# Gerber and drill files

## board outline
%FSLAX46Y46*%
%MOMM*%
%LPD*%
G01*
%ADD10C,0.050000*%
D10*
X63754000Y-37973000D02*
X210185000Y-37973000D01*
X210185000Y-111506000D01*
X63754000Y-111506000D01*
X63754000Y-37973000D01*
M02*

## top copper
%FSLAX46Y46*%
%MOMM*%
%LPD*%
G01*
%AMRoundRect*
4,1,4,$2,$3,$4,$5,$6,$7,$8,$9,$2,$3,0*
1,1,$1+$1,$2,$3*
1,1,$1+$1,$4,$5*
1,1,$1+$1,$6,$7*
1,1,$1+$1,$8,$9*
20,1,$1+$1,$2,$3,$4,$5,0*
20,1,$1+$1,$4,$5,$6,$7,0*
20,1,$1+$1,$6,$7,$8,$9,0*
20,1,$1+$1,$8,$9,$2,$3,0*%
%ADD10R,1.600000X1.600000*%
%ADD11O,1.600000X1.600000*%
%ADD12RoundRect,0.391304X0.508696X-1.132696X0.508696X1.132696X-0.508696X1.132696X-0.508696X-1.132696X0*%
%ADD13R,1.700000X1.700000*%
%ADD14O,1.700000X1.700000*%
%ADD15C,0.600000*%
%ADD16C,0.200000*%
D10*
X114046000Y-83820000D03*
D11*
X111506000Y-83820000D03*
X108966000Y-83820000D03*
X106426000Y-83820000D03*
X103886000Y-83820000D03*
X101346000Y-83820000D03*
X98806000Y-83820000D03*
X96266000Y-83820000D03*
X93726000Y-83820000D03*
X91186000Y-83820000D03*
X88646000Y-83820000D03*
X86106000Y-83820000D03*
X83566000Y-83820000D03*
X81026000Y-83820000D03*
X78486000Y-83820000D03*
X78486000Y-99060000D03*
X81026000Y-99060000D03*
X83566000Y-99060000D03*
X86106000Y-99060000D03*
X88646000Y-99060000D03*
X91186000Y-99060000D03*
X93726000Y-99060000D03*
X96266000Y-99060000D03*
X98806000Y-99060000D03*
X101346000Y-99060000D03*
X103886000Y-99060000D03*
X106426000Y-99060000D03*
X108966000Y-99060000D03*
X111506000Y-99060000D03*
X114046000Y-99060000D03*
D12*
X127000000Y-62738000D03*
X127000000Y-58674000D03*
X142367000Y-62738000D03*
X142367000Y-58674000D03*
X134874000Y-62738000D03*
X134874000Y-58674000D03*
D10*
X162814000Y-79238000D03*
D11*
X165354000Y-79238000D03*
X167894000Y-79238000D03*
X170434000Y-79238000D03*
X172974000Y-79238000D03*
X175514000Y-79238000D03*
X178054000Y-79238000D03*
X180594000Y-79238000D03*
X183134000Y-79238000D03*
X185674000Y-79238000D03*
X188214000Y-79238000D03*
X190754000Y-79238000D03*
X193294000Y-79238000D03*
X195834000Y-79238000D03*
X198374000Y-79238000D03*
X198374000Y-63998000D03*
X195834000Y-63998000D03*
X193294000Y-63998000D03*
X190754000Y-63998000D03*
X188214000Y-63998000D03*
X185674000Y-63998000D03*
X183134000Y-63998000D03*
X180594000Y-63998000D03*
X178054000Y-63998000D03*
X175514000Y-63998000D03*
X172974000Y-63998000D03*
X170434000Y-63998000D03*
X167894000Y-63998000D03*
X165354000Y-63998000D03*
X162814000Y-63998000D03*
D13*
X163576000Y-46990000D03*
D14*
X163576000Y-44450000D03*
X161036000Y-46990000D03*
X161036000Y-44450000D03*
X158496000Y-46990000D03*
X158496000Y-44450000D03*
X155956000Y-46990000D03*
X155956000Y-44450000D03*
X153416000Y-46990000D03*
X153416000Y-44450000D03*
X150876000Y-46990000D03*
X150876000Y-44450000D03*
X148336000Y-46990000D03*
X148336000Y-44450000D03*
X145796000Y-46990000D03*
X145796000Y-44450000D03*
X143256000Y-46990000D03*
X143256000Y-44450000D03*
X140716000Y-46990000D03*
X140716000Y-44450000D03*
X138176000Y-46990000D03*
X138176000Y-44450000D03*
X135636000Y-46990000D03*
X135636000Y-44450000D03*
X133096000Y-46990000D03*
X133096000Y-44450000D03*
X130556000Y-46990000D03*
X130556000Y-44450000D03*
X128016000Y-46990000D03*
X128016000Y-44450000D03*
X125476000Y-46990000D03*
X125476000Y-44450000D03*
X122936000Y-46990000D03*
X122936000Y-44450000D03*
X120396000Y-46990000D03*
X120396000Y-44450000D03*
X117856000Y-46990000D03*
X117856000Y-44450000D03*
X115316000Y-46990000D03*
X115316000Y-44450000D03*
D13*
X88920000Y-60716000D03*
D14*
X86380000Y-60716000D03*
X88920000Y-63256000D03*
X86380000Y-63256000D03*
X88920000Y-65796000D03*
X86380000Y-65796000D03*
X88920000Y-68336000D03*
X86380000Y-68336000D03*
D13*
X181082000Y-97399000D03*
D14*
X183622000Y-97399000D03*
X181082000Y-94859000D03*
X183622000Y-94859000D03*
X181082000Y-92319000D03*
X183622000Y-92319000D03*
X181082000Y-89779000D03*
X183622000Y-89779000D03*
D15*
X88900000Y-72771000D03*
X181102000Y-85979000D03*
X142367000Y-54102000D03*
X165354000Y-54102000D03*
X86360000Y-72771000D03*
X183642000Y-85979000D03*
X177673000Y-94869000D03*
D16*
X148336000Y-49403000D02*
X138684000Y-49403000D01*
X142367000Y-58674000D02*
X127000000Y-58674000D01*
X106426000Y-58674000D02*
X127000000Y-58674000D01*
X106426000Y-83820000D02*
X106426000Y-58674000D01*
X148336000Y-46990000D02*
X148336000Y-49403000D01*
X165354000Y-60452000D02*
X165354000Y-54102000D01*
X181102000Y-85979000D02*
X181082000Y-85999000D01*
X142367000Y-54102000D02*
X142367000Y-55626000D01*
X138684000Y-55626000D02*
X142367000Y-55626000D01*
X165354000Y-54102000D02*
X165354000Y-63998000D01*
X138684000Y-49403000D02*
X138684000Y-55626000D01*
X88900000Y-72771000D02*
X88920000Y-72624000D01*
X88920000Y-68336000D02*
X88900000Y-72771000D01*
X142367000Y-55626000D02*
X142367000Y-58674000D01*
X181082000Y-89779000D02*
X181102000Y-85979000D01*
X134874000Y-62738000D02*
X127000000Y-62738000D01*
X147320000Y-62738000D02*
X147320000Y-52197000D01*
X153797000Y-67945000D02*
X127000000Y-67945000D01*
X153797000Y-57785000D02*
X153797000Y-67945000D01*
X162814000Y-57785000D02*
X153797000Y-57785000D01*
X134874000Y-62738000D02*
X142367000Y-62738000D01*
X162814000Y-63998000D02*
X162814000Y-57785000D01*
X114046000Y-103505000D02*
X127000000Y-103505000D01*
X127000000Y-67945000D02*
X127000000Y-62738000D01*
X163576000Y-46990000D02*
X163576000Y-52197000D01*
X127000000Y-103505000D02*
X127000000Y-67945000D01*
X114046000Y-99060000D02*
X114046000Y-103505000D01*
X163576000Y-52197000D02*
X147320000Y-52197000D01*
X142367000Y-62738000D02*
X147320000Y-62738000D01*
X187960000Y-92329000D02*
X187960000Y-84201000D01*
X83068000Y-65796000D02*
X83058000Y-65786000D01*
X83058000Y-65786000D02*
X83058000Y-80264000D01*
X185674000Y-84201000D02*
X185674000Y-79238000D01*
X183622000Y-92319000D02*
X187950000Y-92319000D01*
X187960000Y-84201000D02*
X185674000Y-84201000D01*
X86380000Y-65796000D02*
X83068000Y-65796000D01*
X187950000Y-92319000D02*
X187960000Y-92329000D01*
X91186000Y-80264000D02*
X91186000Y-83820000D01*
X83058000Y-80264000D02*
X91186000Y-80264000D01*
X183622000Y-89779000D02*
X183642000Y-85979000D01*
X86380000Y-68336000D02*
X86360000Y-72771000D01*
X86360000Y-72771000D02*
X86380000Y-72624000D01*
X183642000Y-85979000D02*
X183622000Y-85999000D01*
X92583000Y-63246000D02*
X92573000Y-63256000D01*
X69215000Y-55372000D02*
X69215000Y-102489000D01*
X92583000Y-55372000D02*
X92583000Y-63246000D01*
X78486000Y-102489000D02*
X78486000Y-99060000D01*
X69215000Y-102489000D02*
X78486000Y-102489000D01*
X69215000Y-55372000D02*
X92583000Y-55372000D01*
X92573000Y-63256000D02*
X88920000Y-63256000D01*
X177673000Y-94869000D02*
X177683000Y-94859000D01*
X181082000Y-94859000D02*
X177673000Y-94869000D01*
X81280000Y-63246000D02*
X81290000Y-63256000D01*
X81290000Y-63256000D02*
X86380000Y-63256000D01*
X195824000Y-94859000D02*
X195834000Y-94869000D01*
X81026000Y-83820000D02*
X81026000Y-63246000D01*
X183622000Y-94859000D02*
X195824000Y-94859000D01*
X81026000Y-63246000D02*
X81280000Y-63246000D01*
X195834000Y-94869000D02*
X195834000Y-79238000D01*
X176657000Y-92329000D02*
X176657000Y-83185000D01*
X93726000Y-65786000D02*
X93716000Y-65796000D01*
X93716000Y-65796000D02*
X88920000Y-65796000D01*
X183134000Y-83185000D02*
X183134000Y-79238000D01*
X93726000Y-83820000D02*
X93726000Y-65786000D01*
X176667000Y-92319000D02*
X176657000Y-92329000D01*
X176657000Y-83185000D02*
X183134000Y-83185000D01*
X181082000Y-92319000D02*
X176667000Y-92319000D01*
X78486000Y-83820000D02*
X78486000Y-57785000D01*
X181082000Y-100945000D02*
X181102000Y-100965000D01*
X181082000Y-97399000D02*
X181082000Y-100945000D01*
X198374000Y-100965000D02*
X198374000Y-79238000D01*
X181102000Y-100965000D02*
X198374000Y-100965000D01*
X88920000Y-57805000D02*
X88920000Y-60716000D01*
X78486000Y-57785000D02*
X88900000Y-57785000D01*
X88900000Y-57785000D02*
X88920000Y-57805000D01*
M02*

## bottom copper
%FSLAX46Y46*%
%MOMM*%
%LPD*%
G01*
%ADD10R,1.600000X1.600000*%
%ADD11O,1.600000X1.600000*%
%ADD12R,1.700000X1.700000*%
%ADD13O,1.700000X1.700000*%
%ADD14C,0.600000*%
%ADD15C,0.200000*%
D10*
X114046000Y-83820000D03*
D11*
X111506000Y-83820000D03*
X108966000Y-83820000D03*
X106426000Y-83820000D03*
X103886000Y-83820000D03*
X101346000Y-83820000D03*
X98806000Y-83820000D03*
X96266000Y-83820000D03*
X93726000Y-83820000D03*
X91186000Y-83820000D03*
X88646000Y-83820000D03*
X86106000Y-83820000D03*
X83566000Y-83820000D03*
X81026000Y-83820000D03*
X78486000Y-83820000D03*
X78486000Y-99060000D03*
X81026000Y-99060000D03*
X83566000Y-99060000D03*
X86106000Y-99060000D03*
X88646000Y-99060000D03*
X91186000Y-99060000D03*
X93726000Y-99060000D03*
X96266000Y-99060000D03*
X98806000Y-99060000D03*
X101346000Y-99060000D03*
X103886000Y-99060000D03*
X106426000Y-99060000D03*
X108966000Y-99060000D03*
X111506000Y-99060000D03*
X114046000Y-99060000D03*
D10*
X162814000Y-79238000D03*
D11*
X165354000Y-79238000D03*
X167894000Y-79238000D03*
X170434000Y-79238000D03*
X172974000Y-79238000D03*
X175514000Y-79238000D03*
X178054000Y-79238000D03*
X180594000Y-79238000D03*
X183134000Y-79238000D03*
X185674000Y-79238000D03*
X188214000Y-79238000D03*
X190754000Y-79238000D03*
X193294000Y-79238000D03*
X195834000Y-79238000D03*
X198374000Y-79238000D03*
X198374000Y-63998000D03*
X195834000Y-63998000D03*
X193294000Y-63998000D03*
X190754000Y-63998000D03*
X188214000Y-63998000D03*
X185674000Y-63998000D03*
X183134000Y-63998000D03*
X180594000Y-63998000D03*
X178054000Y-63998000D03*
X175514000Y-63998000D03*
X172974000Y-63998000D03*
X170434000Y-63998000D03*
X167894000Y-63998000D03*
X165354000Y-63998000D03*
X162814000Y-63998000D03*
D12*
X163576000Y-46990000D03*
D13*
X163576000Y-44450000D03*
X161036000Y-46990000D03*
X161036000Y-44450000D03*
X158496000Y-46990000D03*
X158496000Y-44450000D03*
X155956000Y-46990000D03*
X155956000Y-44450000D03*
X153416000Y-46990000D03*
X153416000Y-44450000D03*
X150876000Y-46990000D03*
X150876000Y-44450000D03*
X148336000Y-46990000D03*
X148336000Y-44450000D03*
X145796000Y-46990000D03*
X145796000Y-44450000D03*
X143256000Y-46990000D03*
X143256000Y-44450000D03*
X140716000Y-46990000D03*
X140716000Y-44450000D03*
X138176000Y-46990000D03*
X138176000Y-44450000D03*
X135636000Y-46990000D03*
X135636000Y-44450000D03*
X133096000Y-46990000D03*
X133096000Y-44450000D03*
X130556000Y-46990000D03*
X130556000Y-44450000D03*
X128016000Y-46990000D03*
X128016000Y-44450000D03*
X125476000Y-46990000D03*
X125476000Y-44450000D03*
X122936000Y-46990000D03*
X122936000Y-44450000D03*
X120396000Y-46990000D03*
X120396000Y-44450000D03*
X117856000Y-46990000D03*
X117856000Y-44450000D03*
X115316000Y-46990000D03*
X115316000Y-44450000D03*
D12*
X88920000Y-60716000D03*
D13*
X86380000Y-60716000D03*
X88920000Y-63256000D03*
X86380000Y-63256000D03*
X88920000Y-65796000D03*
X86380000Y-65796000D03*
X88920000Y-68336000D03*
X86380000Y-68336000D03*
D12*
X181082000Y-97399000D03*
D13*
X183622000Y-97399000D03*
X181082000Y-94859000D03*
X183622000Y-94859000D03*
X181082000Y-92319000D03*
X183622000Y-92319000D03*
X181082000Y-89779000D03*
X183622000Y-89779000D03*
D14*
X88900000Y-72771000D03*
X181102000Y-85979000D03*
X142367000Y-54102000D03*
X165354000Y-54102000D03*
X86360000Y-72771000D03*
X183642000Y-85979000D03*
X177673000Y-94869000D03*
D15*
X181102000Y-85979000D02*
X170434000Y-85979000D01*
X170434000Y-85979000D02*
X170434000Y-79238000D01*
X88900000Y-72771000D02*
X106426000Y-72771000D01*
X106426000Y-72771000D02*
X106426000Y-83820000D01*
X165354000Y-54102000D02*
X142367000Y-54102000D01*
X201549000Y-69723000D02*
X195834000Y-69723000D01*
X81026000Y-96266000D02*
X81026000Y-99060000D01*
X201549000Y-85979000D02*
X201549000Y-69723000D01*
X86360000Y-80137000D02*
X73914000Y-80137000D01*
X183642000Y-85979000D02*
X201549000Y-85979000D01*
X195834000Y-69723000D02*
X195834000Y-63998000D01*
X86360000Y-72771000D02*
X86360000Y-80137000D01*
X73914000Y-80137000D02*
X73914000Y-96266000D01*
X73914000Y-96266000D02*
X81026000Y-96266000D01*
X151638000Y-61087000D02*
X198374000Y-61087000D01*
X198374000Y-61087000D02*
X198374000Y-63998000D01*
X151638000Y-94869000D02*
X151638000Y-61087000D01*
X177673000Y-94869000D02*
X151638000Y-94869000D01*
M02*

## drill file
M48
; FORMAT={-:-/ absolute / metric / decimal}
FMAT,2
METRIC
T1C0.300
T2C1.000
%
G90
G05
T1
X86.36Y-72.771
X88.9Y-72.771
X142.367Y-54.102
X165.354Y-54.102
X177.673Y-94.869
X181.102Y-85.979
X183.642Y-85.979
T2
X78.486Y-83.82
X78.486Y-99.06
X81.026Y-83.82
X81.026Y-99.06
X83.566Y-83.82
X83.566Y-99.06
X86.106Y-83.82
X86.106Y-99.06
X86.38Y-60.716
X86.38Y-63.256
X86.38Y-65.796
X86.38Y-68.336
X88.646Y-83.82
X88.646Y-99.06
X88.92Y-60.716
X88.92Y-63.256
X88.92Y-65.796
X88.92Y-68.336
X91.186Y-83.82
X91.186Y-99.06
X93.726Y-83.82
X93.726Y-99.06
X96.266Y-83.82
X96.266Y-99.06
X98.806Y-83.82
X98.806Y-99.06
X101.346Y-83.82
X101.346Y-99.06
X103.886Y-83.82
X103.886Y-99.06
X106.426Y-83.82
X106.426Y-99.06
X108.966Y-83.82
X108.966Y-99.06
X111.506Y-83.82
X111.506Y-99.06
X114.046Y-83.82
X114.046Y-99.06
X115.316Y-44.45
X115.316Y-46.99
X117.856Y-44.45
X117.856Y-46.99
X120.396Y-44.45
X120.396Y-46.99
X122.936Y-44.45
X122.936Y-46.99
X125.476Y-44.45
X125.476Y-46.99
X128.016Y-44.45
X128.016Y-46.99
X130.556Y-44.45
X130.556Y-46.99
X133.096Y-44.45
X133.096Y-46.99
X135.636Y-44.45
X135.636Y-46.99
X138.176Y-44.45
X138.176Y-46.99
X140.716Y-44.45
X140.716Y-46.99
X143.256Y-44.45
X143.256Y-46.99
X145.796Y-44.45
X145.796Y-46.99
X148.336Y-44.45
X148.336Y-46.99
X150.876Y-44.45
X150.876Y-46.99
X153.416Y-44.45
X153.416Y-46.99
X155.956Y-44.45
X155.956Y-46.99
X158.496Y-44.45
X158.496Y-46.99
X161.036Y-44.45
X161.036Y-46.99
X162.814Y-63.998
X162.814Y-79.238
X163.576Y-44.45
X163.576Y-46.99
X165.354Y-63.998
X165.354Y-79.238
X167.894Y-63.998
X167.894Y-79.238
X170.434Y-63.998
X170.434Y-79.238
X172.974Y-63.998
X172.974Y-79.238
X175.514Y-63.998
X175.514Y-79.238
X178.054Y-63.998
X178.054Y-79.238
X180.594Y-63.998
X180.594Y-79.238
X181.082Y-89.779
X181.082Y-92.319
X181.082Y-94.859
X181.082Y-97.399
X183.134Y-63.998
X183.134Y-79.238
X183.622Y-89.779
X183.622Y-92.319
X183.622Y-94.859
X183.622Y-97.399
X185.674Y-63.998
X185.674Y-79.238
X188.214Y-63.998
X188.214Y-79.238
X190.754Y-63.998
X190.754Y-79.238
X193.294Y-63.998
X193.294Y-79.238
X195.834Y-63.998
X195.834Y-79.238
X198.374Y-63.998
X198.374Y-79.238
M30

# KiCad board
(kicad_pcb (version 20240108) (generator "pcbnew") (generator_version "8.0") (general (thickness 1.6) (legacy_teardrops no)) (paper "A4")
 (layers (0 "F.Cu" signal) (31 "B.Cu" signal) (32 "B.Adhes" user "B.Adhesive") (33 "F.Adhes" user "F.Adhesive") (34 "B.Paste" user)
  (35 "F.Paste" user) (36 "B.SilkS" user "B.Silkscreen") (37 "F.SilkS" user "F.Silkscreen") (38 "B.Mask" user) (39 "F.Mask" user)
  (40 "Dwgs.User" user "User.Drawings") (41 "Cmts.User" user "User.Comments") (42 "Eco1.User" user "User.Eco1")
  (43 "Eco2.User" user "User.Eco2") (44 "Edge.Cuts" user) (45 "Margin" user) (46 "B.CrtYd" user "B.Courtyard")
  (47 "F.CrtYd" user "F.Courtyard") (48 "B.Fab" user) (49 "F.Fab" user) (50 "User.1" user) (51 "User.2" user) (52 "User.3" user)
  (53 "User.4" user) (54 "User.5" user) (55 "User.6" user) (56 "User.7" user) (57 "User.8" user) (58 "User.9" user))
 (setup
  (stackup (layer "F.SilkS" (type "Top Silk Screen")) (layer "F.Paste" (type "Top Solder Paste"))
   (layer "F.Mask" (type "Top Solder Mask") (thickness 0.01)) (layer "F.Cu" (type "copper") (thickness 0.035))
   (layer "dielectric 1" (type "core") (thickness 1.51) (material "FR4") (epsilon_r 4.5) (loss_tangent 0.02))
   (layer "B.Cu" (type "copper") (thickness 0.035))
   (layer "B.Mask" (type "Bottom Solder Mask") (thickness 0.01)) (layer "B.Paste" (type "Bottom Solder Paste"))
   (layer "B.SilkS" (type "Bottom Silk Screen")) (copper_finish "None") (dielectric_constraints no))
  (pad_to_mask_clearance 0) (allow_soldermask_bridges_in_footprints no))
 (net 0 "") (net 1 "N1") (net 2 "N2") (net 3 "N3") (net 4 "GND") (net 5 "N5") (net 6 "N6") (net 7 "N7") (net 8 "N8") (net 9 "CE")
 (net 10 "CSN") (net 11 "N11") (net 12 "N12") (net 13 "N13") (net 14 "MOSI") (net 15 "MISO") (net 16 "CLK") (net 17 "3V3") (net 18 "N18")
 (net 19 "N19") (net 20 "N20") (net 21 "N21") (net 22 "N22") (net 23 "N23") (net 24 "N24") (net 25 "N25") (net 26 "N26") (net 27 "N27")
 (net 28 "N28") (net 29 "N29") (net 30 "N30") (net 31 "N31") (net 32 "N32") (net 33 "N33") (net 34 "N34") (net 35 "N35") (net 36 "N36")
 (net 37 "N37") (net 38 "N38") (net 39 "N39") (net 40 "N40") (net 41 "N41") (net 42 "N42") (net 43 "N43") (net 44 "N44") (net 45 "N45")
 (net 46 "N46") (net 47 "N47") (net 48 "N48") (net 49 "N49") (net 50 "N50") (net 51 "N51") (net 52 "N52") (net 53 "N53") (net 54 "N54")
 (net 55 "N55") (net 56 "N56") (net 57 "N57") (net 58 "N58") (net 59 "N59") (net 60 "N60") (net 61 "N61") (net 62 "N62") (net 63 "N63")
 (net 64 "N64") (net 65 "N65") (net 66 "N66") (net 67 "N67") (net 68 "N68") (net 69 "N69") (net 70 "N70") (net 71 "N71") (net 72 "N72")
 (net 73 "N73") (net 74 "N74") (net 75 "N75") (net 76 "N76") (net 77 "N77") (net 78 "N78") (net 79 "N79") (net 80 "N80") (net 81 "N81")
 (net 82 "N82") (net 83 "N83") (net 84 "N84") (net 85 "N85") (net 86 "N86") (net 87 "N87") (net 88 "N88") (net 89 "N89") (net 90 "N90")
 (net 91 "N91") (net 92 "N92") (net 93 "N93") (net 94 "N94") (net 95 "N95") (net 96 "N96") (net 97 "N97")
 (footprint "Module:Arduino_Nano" (layer "F.Cu") (at 114.046 83.82 -90)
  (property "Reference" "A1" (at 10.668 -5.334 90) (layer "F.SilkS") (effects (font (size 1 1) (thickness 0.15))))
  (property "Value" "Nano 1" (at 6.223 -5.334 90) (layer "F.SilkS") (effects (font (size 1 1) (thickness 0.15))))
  (pad "1" thru_hole rect (at 0 0 270) (size 1.6 1.6) (drill 1) (layers "*.Cu" "*.Mask") (remove_unused_layers no) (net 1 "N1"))
  (pad "2" thru_hole oval (at 0 2.54 270) (size 1.6 1.6) (drill 1) (layers "*.Cu" "*.Mask") (remove_unused_layers no) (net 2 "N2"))
  (pad "3" thru_hole oval (at 0 5.08 270) (size 1.6 1.6) (drill 1) (layers "*.Cu" "*.Mask") (remove_unused_layers no) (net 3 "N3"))
  (pad "4" thru_hole oval (at 0 7.62 270) (size 1.6 1.6) (drill 1) (layers "*.Cu" "*.Mask") (remove_unused_layers no) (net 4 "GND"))
  (pad "5" thru_hole oval (at 0 10.16 270) (size 1.6 1.6) (drill 1) (layers "*.Cu" "*.Mask") (remove_unused_layers no) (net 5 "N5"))
  (pad "6" thru_hole oval (at 0 12.7 270) (size 1.6 1.6) (drill 1) (layers "*.Cu" "*.Mask") (remove_unused_layers no) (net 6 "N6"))
  (pad "7" thru_hole oval (at 0 15.24 270) (size 1.6 1.6) (drill 1) (layers "*.Cu" "*.Mask") (remove_unused_layers no) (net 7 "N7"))
  (pad "8" thru_hole oval (at 0 17.78 270) (size 1.6 1.6) (drill 1) (layers "*.Cu" "*.Mask") (remove_unused_layers no) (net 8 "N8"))
  (pad "9" thru_hole oval (at 0 20.32 270) (size 1.6 1.6) (drill 1) (layers "*.Cu" "*.Mask") (remove_unused_layers no) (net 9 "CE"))
  (pad "10" thru_hole oval (at 0 22.86 270) (size 1.6 1.6) (drill 1) (layers "*.Cu" "*.Mask") (remove_unused_layers no) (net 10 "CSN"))
  (pad "11" thru_hole oval (at 0 25.4 270) (size 1.6 1.6) (drill 1) (layers "*.Cu" "*.Mask") (remove_unused_layers no) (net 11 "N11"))
  (pad "12" thru_hole oval (at 0 27.94 270) (size 1.6 1.6) (drill 1) (layers "*.Cu" "*.Mask") (remove_unused_layers no) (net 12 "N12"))
  (pad "13" thru_hole oval (at 0 30.48 270) (size 1.6 1.6) (drill 1) (layers "*.Cu" "*.Mask") (remove_unused_layers no) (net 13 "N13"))
  (pad "14" thru_hole oval (at 0 33.02 270) (size 1.6 1.6) (drill 1) (layers "*.Cu" "*.Mask") (remove_unused_layers no) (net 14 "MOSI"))
  (pad "15" thru_hole oval (at 0 35.56 270) (size 1.6 1.6) (drill 1) (layers "*.Cu" "*.Mask") (remove_unused_layers no) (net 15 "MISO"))
  (pad "16" thru_hole oval (at 15.24 35.56 270) (size 1.6 1.6) (drill 1) (layers "*.Cu" "*.Mask") (remove_unused_layers no) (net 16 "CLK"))
  (pad "17" thru_hole oval (at 15.24 33.02 270) (size 1.6 1.6) (drill 1) (layers "*.Cu" "*.Mask") (remove_unused_layers no) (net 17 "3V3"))
  (pad "18" thru_hole oval (at 15.24 30.48 270) (size 1.6 1.6) (drill 1) (layers "*.Cu" "*.Mask") (remove_unused_layers no) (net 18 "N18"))
  (pad "19" thru_hole oval (at 15.24 27.94 270) (size 1.6 1.6) (drill 1) (layers "*.Cu" "*.Mask") (remove_unused_layers no) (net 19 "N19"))
  (pad "20" thru_hole oval (at 15.24 25.4 270) (size 1.6 1.6) (drill 1) (layers "*.Cu" "*.Mask") (remove_unused_layers no) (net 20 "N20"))
  (pad "21" thru_hole oval (at 15.24 22.86 270) (size 1.6 1.6) (drill 1) (layers "*.Cu" "*.Mask") (remove_unused_layers no) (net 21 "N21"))
  (pad "22" thru_hole oval (at 15.24 20.32 270) (size 1.6 1.6) (drill 1) (layers "*.Cu" "*.Mask") (remove_unused_layers no) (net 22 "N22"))
  (pad "23" thru_hole oval (at 15.24 17.78 270) (size 1.6 1.6) (drill 1) (layers "*.Cu" "*.Mask") (remove_unused_layers no) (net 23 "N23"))
  (pad "24" thru_hole oval (at 15.24 15.24 270) (size 1.6 1.6) (drill 1) (layers "*.Cu" "*.Mask") (remove_unused_layers no) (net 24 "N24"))
  (pad "25" thru_hole oval (at 15.24 12.7 270) (size 1.6 1.6) (drill 1) (layers "*.Cu" "*.Mask") (remove_unused_layers no) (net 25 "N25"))
  (pad "26" thru_hole oval (at 15.24 10.16 270) (size 1.6 1.6) (drill 1) (layers "*.Cu" "*.Mask") (remove_unused_layers no) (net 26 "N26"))
  (pad "27" thru_hole oval (at 15.24 7.62 270) (size 1.6 1.6) (drill 1) (layers "*.Cu" "*.Mask") (remove_unused_layers no) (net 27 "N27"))
  (pad "28" thru_hole oval (at 15.24 5.08 270) (size 1.6 1.6) (drill 1) (layers "*.Cu" "*.Mask") (remove_unused_layers no) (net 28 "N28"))
  (pad "29" thru_hole oval (at 15.24 2.54 270) (size 1.6 1.6) (drill 1) (layers "*.Cu" "*.Mask") (remove_unused_layers no) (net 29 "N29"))
  (pad "30" thru_hole oval (at 15.24 0 270) (size 1.6 1.6) (drill 1) (layers "*.Cu" "*.Mask") (remove_unused_layers no) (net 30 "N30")))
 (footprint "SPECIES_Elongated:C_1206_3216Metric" (layer "F.Cu") (at 127 60.706 90)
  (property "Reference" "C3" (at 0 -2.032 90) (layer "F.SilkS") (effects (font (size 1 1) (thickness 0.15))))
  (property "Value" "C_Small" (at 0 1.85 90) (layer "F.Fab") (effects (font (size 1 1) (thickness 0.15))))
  (pad "1" smd roundrect (at -2.032 0 90) (size 3.048 1.8) (layers "F.Cu" "F.Paste" "F.Mask") (roundrect_rratio 0.217391) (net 30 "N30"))
  (pad "2" smd roundrect (at 2.032 0 90) (size 3.048 1.8) (layers "F.Cu" "F.Paste" "F.Mask") (roundrect_rratio 0.217391) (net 4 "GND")))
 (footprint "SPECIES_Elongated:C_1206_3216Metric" (layer "F.Cu") (at 142.367 60.706 90)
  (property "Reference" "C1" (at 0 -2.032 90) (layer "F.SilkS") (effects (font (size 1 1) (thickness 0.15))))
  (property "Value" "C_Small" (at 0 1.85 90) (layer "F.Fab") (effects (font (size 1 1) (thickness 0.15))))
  (pad "1" smd roundrect (at -2.032 0 90) (size 3.048 1.8) (layers "F.Cu" "F.Paste" "F.Mask") (roundrect_rratio 0.217391) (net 30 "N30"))
  (pad "2" smd roundrect (at 2.032 0 90) (size 3.048 1.8) (layers "F.Cu" "F.Paste" "F.Mask") (roundrect_rratio 0.217391) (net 4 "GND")))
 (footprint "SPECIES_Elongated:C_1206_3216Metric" (layer "F.Cu") (at 134.874 60.706 90)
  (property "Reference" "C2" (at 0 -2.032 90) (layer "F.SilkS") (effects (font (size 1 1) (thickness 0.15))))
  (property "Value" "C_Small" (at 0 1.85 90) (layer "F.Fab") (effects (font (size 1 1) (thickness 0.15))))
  (pad "1" smd roundrect (at -2.032 0 90) (size 3.048 1.8) (layers "F.Cu" "F.Paste" "F.Mask") (roundrect_rratio 0.217391) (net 30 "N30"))
  (pad "2" smd roundrect (at 2.032 0 90) (size 3.048 1.8) (layers "F.Cu" "F.Paste" "F.Mask") (roundrect_rratio 0.217391) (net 4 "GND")))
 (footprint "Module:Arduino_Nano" (layer "F.Cu") (at 162.814 79.238 90)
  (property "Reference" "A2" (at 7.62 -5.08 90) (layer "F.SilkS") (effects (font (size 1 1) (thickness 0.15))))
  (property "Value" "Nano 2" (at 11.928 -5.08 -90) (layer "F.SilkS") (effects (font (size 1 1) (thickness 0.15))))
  (pad "1" thru_hole rect (at 0 0 90) (size 1.6 1.6) (drill 1) (layers "*.Cu" "*.Mask") (remove_unused_layers no) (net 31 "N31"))
  (pad "2" thru_hole oval (at 0 2.54 90) (size 1.6 1.6) (drill 1) (layers "*.Cu" "*.Mask") (remove_unused_layers no) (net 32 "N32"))
  (pad "3" thru_hole oval (at 0 5.08 90) (size 1.6 1.6) (drill 1) (layers "*.Cu" "*.Mask") (remove_unused_layers no) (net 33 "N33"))
  (pad "4" thru_hole oval (at 0 7.62 90) (size 1.6 1.6) (drill 1) (layers "*.Cu" "*.Mask") (remove_unused_layers no) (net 4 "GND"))
  (pad "5" thru_hole oval (at 0 10.16 90) (size 1.6 1.6) (drill 1) (layers "*.Cu" "*.Mask") (remove_unused_layers no) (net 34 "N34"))
  (pad "6" thru_hole oval (at 0 12.7 90) (size 1.6 1.6) (drill 1) (layers "*.Cu" "*.Mask") (remove_unused_layers no) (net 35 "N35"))
  (pad "7" thru_hole oval (at 0 15.24 90) (size 1.6 1.6) (drill 1) (layers "*.Cu" "*.Mask") (remove_unused_layers no) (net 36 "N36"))
  (pad "8" thru_hole oval (at 0 17.78 90) (size 1.6 1.6) (drill 1) (layers "*.Cu" "*.Mask") (remove_unused_layers no) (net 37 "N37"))
  (pad "9" thru_hole oval (at 0 20.32 90) (size 1.6 1.6) (drill 1) (layers "*.Cu" "*.Mask") (remove_unused_layers no) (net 9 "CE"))
  (pad "10" thru_hole oval (at 0 22.86 90) (size 1.6 1.6) (drill 1) (layers "*.Cu" "*.Mask") (remove_unused_layers no) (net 10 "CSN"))
  (pad "11" thru_hole oval (at 0 25.4 90) (size 1.6 1.6) (drill 1) (layers "*.Cu" "*.Mask") (remove_unused_layers no) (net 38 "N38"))
  (pad "12" thru_hole oval (at 0 27.94 90) (size 1.6 1.6) (drill 1) (layers "*.Cu" "*.Mask") (remove_unused_layers no) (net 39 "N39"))
  (pad "13" thru_hole oval (at 0 30.48 90) (size 1.6 1.6) (drill 1) (layers "*.Cu" "*.Mask") (remove_unused_layers no) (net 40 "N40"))
  (pad "14" thru_hole oval (at 0 33.02 90) (size 1.6 1.6) (drill 1) (layers "*.Cu" "*.Mask") (remove_unused_layers no) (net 14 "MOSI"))
  (pad "15" thru_hole oval (at 0 35.56 90) (size 1.6 1.6) (drill 1) (layers "*.Cu" "*.Mask") (remove_unused_layers no) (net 15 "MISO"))
  (pad "16" thru_hole oval (at 15.24 35.56 90) (size 1.6 1.6) (drill 1) (layers "*.Cu" "*.Mask") (remove_unused_layers no) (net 16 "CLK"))
  (pad "17" thru_hole oval (at 15.24 33.02 90) (size 1.6 1.6) (drill 1) (layers "*.Cu" "*.Mask") (remove_unused_layers no) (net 17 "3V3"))
  (pad "18" thru_hole oval (at 15.24 30.48 90) (size 1.6 1.6) (drill 1) (layers "*.Cu" "*.Mask") (remove_unused_layers no) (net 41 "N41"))
  (pad "19" thru_hole oval (at 15.24 27.94 90) (size 1.6 1.6) (drill 1) (layers "*.Cu" "*.Mask") (remove_unused_layers no) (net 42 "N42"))
  (pad "20" thru_hole oval (at 15.24 25.4 90) (size 1.6 1.6) (drill 1) (layers "*.Cu" "*.Mask") (remove_unused_layers no) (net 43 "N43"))
  (pad "21" thru_hole oval (at 15.24 22.86 90) (size 1.6 1.6) (drill 1) (layers "*.Cu" "*.Mask") (remove_unused_layers no) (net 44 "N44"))
  (pad "22" thru_hole oval (at 15.24 20.32 90) (size 1.6 1.6) (drill 1) (layers "*.Cu" "*.Mask") (remove_unused_layers no) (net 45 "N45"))
  (pad "23" thru_hole oval (at 15.24 17.78 90) (size 1.6 1.6) (drill 1) (layers "*.Cu" "*.Mask") (remove_unused_layers no) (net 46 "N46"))
  (pad "24" thru_hole oval (at 15.24 15.24 90) (size 1.6 1.6) (drill 1) (layers "*.Cu" "*.Mask") (remove_unused_layers no) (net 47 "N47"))
  (pad "25" thru_hole oval (at 15.24 12.7 90) (size 1.6 1.6) (drill 1) (layers "*.Cu" "*.Mask") (remove_unused_layers no) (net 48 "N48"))
  (pad "26" thru_hole oval (at 15.24 10.16 90) (size 1.6 1.6) (drill 1) (layers "*.Cu" "*.Mask") (remove_unused_layers no) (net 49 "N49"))
  (pad "27" thru_hole oval (at 15.24 7.62 90) (size 1.6 1.6) (drill 1) (layers "*.Cu" "*.Mask") (remove_unused_layers no) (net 30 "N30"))
  (pad "28" thru_hole oval (at 15.24 5.08 90) (size 1.6 1.6) (drill 1) (layers "*.Cu" "*.Mask") (remove_unused_layers no) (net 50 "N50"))
  (pad "29" thru_hole oval (at 15.24 2.54 90) (size 1.6 1.6) (drill 1) (layers "*.Cu" "*.Mask") (remove_unused_layers no) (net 4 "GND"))
  (pad "30" thru_hole oval (at 15.24 0 90) (size 1.6 1.6) (drill 1) (layers "*.Cu" "*.Mask") (remove_unused_layers no) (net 30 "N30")))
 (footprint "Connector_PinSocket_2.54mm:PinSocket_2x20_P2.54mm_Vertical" (layer "F.Cu") (at 163.576 46.99 -90)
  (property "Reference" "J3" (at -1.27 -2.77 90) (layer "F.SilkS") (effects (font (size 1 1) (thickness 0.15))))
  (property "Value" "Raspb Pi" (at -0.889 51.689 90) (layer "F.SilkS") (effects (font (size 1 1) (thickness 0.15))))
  (pad "1" thru_hole rect (at 0 0 270) (size 1.7 1.7) (drill 1) (layers "*.Cu" "*.Mask") (remove_unused_layers no) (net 30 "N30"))
  (pad "2" thru_hole oval (at -2.54 0 270) (size 1.7 1.7) (drill 1) (layers "*.Cu" "*.Mask") (remove_unused_layers no) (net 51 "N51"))
  (pad "3" thru_hole oval (at 0 2.54 270) (size 1.7 1.7) (drill 1) (layers "*.Cu" "*.Mask") (remove_unused_layers no) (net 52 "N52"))
  (pad "4" thru_hole oval (at -2.54 2.54 270) (size 1.7 1.7) (drill 1) (layers "*.Cu" "*.Mask") (remove_unused_layers no) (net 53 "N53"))
  (pad "5" thru_hole oval (at 0 5.08 270) (size 1.7 1.7) (drill 1) (layers "*.Cu" "*.Mask") (remove_unused_layers no) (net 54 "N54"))
  (pad "6" thru_hole oval (at -2.54 5.08 270) (size 1.7 1.7) (drill 1) (layers "*.Cu" "*.Mask") (remove_unused_layers no) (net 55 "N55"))
  (pad "7" thru_hole oval (at 0 7.62 270) (size 1.7 1.7) (drill 1) (layers "*.Cu" "*.Mask") (remove_unused_layers no) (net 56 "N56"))
  (pad "8" thru_hole oval (at -2.54 7.62 270) (size 1.7 1.7) (drill 1) (layers "*.Cu" "*.Mask") (remove_unused_layers no) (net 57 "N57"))
  (pad "9" thru_hole oval (at 0 10.16 270) (size 1.7 1.7) (drill 1) (layers "*.Cu" "*.Mask") (remove_unused_layers no) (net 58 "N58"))
  (pad "10" thru_hole oval (at -2.54 10.16 270) (size 1.7 1.7) (drill 1) (layers "*.Cu" "*.Mask") (remove_unused_layers no) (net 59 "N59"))
  (pad "11" thru_hole oval (at 0 12.7 270) (size 1.7 1.7) (drill 1) (layers "*.Cu" "*.Mask") (remove_unused_layers no) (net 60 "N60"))
  (pad "12" thru_hole oval (at -2.54 12.7 270) (size 1.7 1.7) (drill 1) (layers "*.Cu" "*.Mask") (remove_unused_layers no) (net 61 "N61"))
  (pad "13" thru_hole oval (at 0 15.24 270) (size 1.7 1.7) (drill 1) (layers "*.Cu" "*.Mask") (remove_unused_layers no) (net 4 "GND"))
  (pad "14" thru_hole oval (at -2.54 15.24 270) (size 1.7 1.7) (drill 1) (layers "*.Cu" "*.Mask") (remove_unused_layers no) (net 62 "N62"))
  (pad "15" thru_hole oval (at 0 17.78 270) (size 1.7 1.7) (drill 1) (layers "*.Cu" "*.Mask") (remove_unused_layers no) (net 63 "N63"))
  (pad "16" thru_hole oval (at -2.54 17.78 270) (size 1.7 1.7) (drill 1) (layers "*.Cu" "*.Mask") (remove_unused_layers no) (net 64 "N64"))
  (pad "17" thru_hole oval (at 0 20.32 270) (size 1.7 1.7) (drill 1) (layers "*.Cu" "*.Mask") (remove_unused_layers no) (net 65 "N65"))
  (pad "18" thru_hole oval (at -2.54 20.32 270) (size 1.7 1.7) (drill 1) (layers "*.Cu" "*.Mask") (remove_unused_layers no) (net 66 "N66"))
  (pad "19" thru_hole oval (at 0 22.86 270) (size 1.7 1.7) (drill 1) (layers "*.Cu" "*.Mask") (remove_unused_layers no) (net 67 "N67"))
  (pad "20" thru_hole oval (at -2.54 22.86 270) (size 1.7 1.7) (drill 1) (layers "*.Cu" "*.Mask") (remove_unused_layers no) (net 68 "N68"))
  (pad "21" thru_hole oval (at 0 25.4 270) (size 1.7 1.7) (drill 1) (layers "*.Cu" "*.Mask") (remove_unused_layers no) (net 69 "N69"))
  (pad "22" thru_hole oval (at -2.54 25.4 270) (size 1.7 1.7) (drill 1) (layers "*.Cu" "*.Mask") (remove_unused_layers no) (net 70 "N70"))
  (pad "23" thru_hole oval (at 0 27.94 270) (size 1.7 1.7) (drill 1) (layers "*.Cu" "*.Mask") (remove_unused_layers no) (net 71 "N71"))
  (pad "24" thru_hole oval (at -2.54 27.94 270) (size 1.7 1.7) (drill 1) (layers "*.Cu" "*.Mask") (remove_unused_layers no) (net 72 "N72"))
  (pad "25" thru_hole oval (at 0 30.48 270) (size 1.7 1.7) (drill 1) (layers "*.Cu" "*.Mask") (remove_unused_layers no) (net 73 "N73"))
  (pad "26" thru_hole oval (at -2.54 30.48 270) (size 1.7 1.7) (drill 1) (layers "*.Cu" "*.Mask") (remove_unused_layers no) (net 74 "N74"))
  (pad "27" thru_hole oval (at 0 33.02 270) (size 1.7 1.7) (drill 1) (layers "*.Cu" "*.Mask") (remove_unused_layers no) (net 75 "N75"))
  (pad "28" thru_hole oval (at -2.54 33.02 270) (size 1.7 1.7) (drill 1) (layers "*.Cu" "*.Mask") (remove_unused_layers no) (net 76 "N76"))
  (pad "29" thru_hole oval (at 0 35.56 270) (size 1.7 1.7) (drill 1) (layers "*.Cu" "*.Mask") (remove_unused_layers no) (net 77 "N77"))
  (pad "30" thru_hole oval (at -2.54 35.56 270) (size 1.7 1.7) (drill 1) (layers "*.Cu" "*.Mask") (remove_unused_layers no) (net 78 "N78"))
  (pad "31" thru_hole oval (at 0 38.1 270) (size 1.7 1.7) (drill 1) (layers "*.Cu" "*.Mask") (remove_unused_layers no) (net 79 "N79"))
  (pad "32" thru_hole oval (at -2.54 38.1 270) (size 1.7 1.7) (drill 1) (layers "*.Cu" "*.Mask") (remove_unused_layers no) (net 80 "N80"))
  (pad "33" thru_hole oval (at 0 40.64 270) (size 1.7 1.7) (drill 1) (layers "*.Cu" "*.Mask") (remove_unused_layers no) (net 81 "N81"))
  (pad "34" thru_hole oval (at -2.54 40.64 270) (size 1.7 1.7) (drill 1) (layers "*.Cu" "*.Mask") (remove_unused_layers no) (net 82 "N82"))
  (pad "35" thru_hole oval (at 0 43.18 270) (size 1.7 1.7) (drill 1) (layers "*.Cu" "*.Mask") (remove_unused_layers no) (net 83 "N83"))
  (pad "36" thru_hole oval (at -2.54 43.18 270) (size 1.7 1.7) (drill 1) (layers "*.Cu" "*.Mask") (remove_unused_layers no) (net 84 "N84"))
  (pad "37" thru_hole oval (at 0 45.72 270) (size 1.7 1.7) (drill 1) (layers "*.Cu" "*.Mask") (remove_unused_layers no) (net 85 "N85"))
  (pad "38" thru_hole oval (at -2.54 45.72 270) (size 1.7 1.7) (drill 1) (layers "*.Cu" "*.Mask") (remove_unused_layers no) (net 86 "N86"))
  (pad "39" thru_hole oval (at 0 48.26 270) (size 1.7 1.7) (drill 1) (layers "*.Cu" "*.Mask") (remove_unused_layers no) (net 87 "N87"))
  (pad "40" thru_hole oval (at -2.54 48.26 270) (size 1.7 1.7) (drill 1) (layers "*.Cu" "*.Mask") (remove_unused_layers no) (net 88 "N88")))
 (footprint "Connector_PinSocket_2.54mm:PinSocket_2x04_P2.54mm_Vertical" (layer "F.Cu") (at 88.92 60.716)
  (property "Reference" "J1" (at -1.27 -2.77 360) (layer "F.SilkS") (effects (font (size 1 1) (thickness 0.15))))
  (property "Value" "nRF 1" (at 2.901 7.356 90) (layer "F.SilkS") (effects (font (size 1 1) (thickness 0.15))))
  (pad "1" thru_hole rect (at 0 0) (size 1.7 1.7) (drill 1) (layers "*.Cu" "*.Mask") (remove_unused_layers no) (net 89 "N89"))
  (pad "2" thru_hole oval (at -2.54 0) (size 1.7 1.7) (drill 1) (layers "*.Cu" "*.Mask") (remove_unused_layers no) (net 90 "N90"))
  (pad "3" thru_hole oval (at 0 2.54) (size 1.7 1.7) (drill 1) (layers "*.Cu" "*.Mask") (remove_unused_layers no) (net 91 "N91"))
  (pad "4" thru_hole oval (at -2.54 2.54) (size 1.7 1.7) (drill 1) (layers "*.Cu" "*.Mask") (remove_unused_layers no) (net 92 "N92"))
  (pad "5" thru_hole oval (at 0 5.08) (size 1.7 1.7) (drill 1) (layers "*.Cu" "*.Mask") (remove_unused_layers no) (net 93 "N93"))
  (pad "6" thru_hole oval (at -2.54 5.08) (size 1.7 1.7) (drill 1) (layers "*.Cu" "*.Mask") (remove_unused_layers no) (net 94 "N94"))
  (pad "7" thru_hole oval (at 0 7.62) (size 1.7 1.7) (drill 1) (layers "*.Cu" "*.Mask") (remove_unused_layers no) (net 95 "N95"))
  (pad "8" thru_hole oval (at -2.54 7.62) (size 1.7 1.7) (drill 1) (layers "*.Cu" "*.Mask") (remove_unused_layers no) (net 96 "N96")))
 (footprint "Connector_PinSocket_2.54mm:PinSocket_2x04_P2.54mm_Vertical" (layer "F.Cu") (at 181.082 97.399 180)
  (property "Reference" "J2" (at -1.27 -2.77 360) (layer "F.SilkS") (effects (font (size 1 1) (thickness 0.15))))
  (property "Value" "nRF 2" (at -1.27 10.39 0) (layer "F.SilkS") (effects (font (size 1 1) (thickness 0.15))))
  (pad "1" thru_hole rect (at 0 0 180) (size 1.7 1.7) (drill 1) (layers "*.Cu" "*.Mask") (remove_unused_layers no) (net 15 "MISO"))
  (pad "2" thru_hole oval (at -2.54 0 180) (size 1.7 1.7) (drill 1) (layers "*.Cu" "*.Mask") (remove_unused_layers no) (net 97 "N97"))
  (pad "3" thru_hole oval (at 0 2.54 180) (size 1.7 1.7) (drill 1) (layers "*.Cu" "*.Mask") (remove_unused_layers no) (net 16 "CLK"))
  (pad "4" thru_hole oval (at -2.54 2.54 180) (size 1.7 1.7) (drill 1) (layers "*.Cu" "*.Mask") (remove_unused_layers no) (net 14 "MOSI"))
  (pad "5" thru_hole oval (at 0 5.08 180) (size 1.7 1.7) (drill 1) (layers "*.Cu" "*.Mask") (remove_unused_layers no) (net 9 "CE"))
  (pad "6" thru_hole oval (at -2.54 5.08 180) (size 1.7 1.7) (drill 1) (layers "*.Cu" "*.Mask") (remove_unused_layers no) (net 10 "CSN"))
  (pad "7" thru_hole oval (at 0 7.62 180) (size 1.7 1.7) (drill 1) (layers "*.Cu" "*.Mask") (remove_unused_layers no) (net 4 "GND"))
  (pad "8" thru_hole oval (at -2.54 7.62 180) (size 1.7 1.7) (drill 1) (layers "*.Cu" "*.Mask") (remove_unused_layers no) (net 17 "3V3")))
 (gr_rect (start 63.754 37.973) (end 210.185 111.506) (stroke (width 0.05) (type default)) (fill none) (layer "Edge.Cuts"))
 (segment (start 148.336 49.403) (end 138.684 49.403) (width 0.2) (layer "F.Cu") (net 4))
 (segment (start 142.367 58.674) (end 127 58.674) (width 0.2) (layer "F.Cu") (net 4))
 (segment (start 106.426 58.674) (end 127 58.674) (width 0.2) (layer "F.Cu") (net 4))
 (segment (start 106.426 83.82) (end 106.426 58.674) (width 0.2) (layer "F.Cu") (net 4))
 (segment (start 148.336 46.99) (end 148.336 49.403) (width 0.2) (layer "F.Cu") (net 4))
 (segment (start 165.354 60.452) (end 165.354 54.102) (width 0.2) (layer "F.Cu") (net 4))
 (segment (start 181.102 85.979) (end 181.082 85.999) (width 0.2) (layer "F.Cu") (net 4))
 (segment (start 142.367 54.102) (end 142.367 55.626) (width 0.2) (layer "F.Cu") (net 4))
 (segment (start 138.684 55.626) (end 142.367 55.626) (width 0.2) (layer "F.Cu") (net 4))
 (segment (start 165.354 54.102) (end 165.354 63.998) (width 0.2) (layer "F.Cu") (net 4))
 (segment (start 138.684 49.403) (end 138.684 55.626) (width 0.2) (layer "F.Cu") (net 4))
 (segment (start 88.9 72.771) (end 88.92 72.624) (width 0.2) (layer "F.Cu") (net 4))
 (segment (start 88.92 68.336) (end 88.9 72.771) (width 0.2) (layer "F.Cu") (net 4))
 (segment (start 142.367 55.626) (end 142.367 58.674) (width 0.2) (layer "F.Cu") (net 4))
 (segment (start 181.082 89.779) (end 181.102 85.979) (width 0.2) (layer "F.Cu") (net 4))
 (via (at 88.9 72.771) (size 0.6) (drill 0.3) (layers "F.Cu" "B.Cu") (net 4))
 (via (at 181.102 85.979) (size 0.6) (drill 0.3) (layers "F.Cu" "B.Cu") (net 4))
 (via (at 142.367 54.102) (size 0.6) (drill 0.3) (layers "F.Cu" "B.Cu") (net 4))
 (via (at 165.354 54.102) (size 0.6) (drill 0.3) (layers "F.Cu" "B.Cu") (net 4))
 (segment (start 181.102 85.979) (end 170.434 85.979) (width 0.2) (layer "B.Cu") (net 4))
 (segment (start 170.434 85.979) (end 170.434 79.238) (width 0.2) (layer "B.Cu") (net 4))
 (segment (start 88.9 72.771) (end 106.426 72.771) (width 0.2) (layer "B.Cu") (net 4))
 (segment (start 106.426 72.771) (end 106.426 83.82) (width 0.2) (layer "B.Cu") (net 4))
 (segment (start 165.354 54.102) (end 142.367 54.102) (width 0.2) (layer "B.Cu") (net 4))
 (segment (start 134.874 62.738) (end 127 62.738) (width 0.2) (layer "F.Cu") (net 30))
 (segment (start 147.32 62.738) (end 147.32 52.197) (width 0.2) (layer "F.Cu") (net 30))
 (segment (start 153.797 67.945) (end 127 67.945) (width 0.2) (layer "F.Cu") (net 30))
 (segment (start 153.797 57.785) (end 153.797 67.945) (width 0.2) (layer "F.Cu") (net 30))
 (segment (start 162.814 57.785) (end 153.797 57.785) (width 0.2) (layer "F.Cu") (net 30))
 (segment (start 134.874 62.738) (end 142.367 62.738) (width 0.2) (layer "F.Cu") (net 30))
 (segment (start 162.814 63.998) (end 162.814 57.785) (width 0.2) (layer "F.Cu") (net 30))
 (segment (start 114.046 103.505) (end 127 103.505) (width 0.2) (layer "F.Cu") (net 30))
 (segment (start 127 67.945) (end 127 62.738) (width 0.2) (layer "F.Cu") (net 30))
 (segment (start 163.576 46.99) (end 163.576 52.197) (width 0.2) (layer "F.Cu") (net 30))
 (segment (start 127 103.505) (end 127 67.945) (width 0.2) (layer "F.Cu") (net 30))
 (segment (start 114.046 99.06) (end 114.046 103.505) (width 0.2) (layer "F.Cu") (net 30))
 (segment (start 163.576 52.197) (end 147.32 52.197) (width 0.2) (layer "F.Cu") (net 30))
 (segment (start 142.367 62.738) (end 147.32 62.738) (width 0.2) (layer "F.Cu") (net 30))
 (segment (start 187.96 92.329) (end 187.96 84.201) (width 0.2) (layer "F.Cu") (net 10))
 (segment (start 83.068 65.796) (end 83.058 65.786) (width 0.2) (layer "F.Cu") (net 10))
 (segment (start 83.058 65.786) (end 83.058 80.264) (width 0.2) (layer "F.Cu") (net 10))
 (segment (start 185.674 84.201) (end 185.674 79.238) (width 0.2) (layer "F.Cu") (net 10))
 (segment (start 183.622 92.319) (end 187.95 92.319) (width 0.2) (layer "F.Cu") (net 10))
 (segment (start 187.96 84.201) (end 185.674 84.201) (width 0.2) (layer "F.Cu") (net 10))
 (segment (start 86.38 65.796) (end 83.068 65.796) (width 0.2) (layer "F.Cu") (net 10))
 (segment (start 187.95 92.319) (end 187.96 92.329) (width 0.2) (layer "F.Cu") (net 10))
 (segment (start 91.186 80.264) (end 91.186 83.82) (width 0.2) (layer "F.Cu") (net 10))
 (segment (start 83.058 80.264) (end 91.186 80.264) (width 0.2) (layer "F.Cu") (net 10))
 (segment (start 183.622 89.779) (end 183.642 85.979) (width 0.2) (layer "F.Cu") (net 17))
 (segment (start 86.38 68.336) (end 86.36 72.771) (width 0.2) (layer "F.Cu") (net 17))
 (segment (start 86.36 72.771) (end 86.38 72.624) (width 0.2) (layer "F.Cu") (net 17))
 (segment (start 183.642 85.979) (end 183.622 85.999) (width 0.2) (layer "F.Cu") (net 17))
 (via (at 86.36 72.771) (size 0.6) (drill 0.3) (layers "F.Cu" "B.Cu") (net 17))
 (via (at 183.642 85.979) (size 0.6) (drill 0.3) (layers "F.Cu" "B.Cu") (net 17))
 (segment (start 201.549 69.723) (end 195.834 69.723) (width 0.2) (layer "B.Cu") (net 17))
 (segment (start 81.026 96.266) (end 81.026 99.06) (width 0.2) (layer "B.Cu") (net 17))
 (segment (start 201.549 85.979) (end 201.549 69.723) (width 0.2) (layer "B.Cu") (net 17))
 (segment (start 86.36 80.137) (end 73.914 80.137) (width 0.2) (layer "B.Cu") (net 17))
 (segment (start 183.642 85.979) (end 201.549 85.979) (width 0.2) (layer "B.Cu") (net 17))
 (segment (start 195.834 69.723) (end 195.834 63.998) (width 0.2) (layer "B.Cu") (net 17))
 (segment (start 86.36 72.771) (end 86.36 80.137) (width 0.2) (layer "B.Cu") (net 17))
 (segment (start 73.914 80.137) (end 73.914 96.266) (width 0.2) (layer "B.Cu") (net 17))
 (segment (start 73.914 96.266) (end 81.026 96.266) (width 0.2) (layer "B.Cu") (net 17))
 (segment (start 92.583 63.246) (end 92.573 63.256) (width 0.2) (layer "F.Cu") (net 16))
 (segment (start 69.215 55.372) (end 69.215 102.489) (width 0.2) (layer "F.Cu") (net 16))
 (segment (start 92.583 55.372) (end 92.583 63.246) (width 0.2) (layer "F.Cu") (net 16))
 (segment (start 78.486 102.489) (end 78.486 99.06) (width 0.2) (layer "F.Cu") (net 16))
 (segment (start 69.215 102.489) (end 78.486 102.489) (width 0.2) (layer "F.Cu") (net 16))
 (segment (start 69.215 55.372) (end 92.583 55.372) (width 0.2) (layer "F.Cu") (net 16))
 (segment (start 92.573 63.256) (end 88.92 63.256) (width 0.2) (layer "F.Cu") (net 16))
 (segment (start 177.673 94.869) (end 177.683 94.859) (width 0.2) (layer "F.Cu") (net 16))
 (segment (start 181.082 94.859) (end 177.673 94.869) (width 0.2) (layer "F.Cu") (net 16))
 (via (at 177.673 94.869) (size 0.6) (drill 0.3) (layers "F.Cu" "B.Cu") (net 16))
 (segment (start 151.638 61.087) (end 198.374 61.087) (width 0.2) (layer "B.Cu") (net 16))
 (segment (start 198.374 61.087) (end 198.374 63.998) (width 0.2) (layer "B.Cu") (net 16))
 (segment (start 151.638 94.869) (end 151.638 61.087) (width 0.2) (layer "B.Cu") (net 16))
 (segment (start 177.673 94.869) (end 151.638 94.869) (width 0.2) (layer "B.Cu") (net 16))
 (segment (start 81.28 63.246) (end 81.29 63.256) (width 0.2) (layer "F.Cu") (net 14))
 (segment (start 81.29 63.256) (end 86.38 63.256) (width 0.2) (layer "F.Cu") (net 14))
 (segment (start 195.824 94.859) (end 195.834 94.869) (width 0.2) (layer "F.Cu") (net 14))
 (segment (start 81.026 83.82) (end 81.026 63.246) (width 0.2) (layer "F.Cu") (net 14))
 (segment (start 183.622 94.859) (end 195.824 94.859) (width 0.2) (layer "F.Cu") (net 14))
 (segment (start 81.026 63.246) (end 81.28 63.246) (width 0.2) (layer "F.Cu") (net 14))
 (segment (start 195.834 94.869) (end 195.834 79.238) (width 0.2) (layer "F.Cu") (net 14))
 (segment (start 176.657 92.329) (end 176.657 83.185) (width 0.2) (layer "F.Cu") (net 9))
 (segment (start 93.726 65.786) (end 93.716 65.796) (width 0.2) (layer "F.Cu") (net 9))
 (segment (start 93.716 65.796) (end 88.92 65.796) (width 0.2) (layer "F.Cu") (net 9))
 (segment (start 183.134 83.185) (end 183.134 79.238) (width 0.2) (layer "F.Cu") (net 9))
 (segment (start 93.726 83.82) (end 93.726 65.786) (width 0.2) (layer "F.Cu") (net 9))
 (segment (start 176.667 92.319) (end 176.657 92.329) (width 0.2) (layer "F.Cu") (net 9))
 (segment (start 176.657 83.185) (end 183.134 83.185) (width 0.2) (layer "F.Cu") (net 9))
 (segment (start 181.082 92.319) (end 176.667 92.319) (width 0.2) (layer "F.Cu") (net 9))
 (segment (start 78.486 83.82) (end 78.486 57.785) (width 0.2) (layer "F.Cu") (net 15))
 (segment (start 181.082 100.945) (end 181.102 100.965) (width 0.2) (layer "F.Cu") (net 15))
 (segment (start 181.082 97.399) (end 181.082 100.945) (width 0.2) (layer "F.Cu") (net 15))
 (segment (start 198.374 100.965) (end 198.374 79.238) (width 0.2) (layer "F.Cu") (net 15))
 (segment (start 181.102 100.965) (end 198.374 100.965) (width 0.2) (layer "F.Cu") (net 15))
 (segment (start 88.92 57.805) (end 88.92 60.716) (width 0.2) (layer "F.Cu") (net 15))
 (segment (start 78.486 57.785) (end 88.9 57.785) (width 0.2) (layer "F.Cu") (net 15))
 (segment (start 88.9 57.785) (end 88.92 57.805) (width 0.2) (layer "F.Cu") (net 15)))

